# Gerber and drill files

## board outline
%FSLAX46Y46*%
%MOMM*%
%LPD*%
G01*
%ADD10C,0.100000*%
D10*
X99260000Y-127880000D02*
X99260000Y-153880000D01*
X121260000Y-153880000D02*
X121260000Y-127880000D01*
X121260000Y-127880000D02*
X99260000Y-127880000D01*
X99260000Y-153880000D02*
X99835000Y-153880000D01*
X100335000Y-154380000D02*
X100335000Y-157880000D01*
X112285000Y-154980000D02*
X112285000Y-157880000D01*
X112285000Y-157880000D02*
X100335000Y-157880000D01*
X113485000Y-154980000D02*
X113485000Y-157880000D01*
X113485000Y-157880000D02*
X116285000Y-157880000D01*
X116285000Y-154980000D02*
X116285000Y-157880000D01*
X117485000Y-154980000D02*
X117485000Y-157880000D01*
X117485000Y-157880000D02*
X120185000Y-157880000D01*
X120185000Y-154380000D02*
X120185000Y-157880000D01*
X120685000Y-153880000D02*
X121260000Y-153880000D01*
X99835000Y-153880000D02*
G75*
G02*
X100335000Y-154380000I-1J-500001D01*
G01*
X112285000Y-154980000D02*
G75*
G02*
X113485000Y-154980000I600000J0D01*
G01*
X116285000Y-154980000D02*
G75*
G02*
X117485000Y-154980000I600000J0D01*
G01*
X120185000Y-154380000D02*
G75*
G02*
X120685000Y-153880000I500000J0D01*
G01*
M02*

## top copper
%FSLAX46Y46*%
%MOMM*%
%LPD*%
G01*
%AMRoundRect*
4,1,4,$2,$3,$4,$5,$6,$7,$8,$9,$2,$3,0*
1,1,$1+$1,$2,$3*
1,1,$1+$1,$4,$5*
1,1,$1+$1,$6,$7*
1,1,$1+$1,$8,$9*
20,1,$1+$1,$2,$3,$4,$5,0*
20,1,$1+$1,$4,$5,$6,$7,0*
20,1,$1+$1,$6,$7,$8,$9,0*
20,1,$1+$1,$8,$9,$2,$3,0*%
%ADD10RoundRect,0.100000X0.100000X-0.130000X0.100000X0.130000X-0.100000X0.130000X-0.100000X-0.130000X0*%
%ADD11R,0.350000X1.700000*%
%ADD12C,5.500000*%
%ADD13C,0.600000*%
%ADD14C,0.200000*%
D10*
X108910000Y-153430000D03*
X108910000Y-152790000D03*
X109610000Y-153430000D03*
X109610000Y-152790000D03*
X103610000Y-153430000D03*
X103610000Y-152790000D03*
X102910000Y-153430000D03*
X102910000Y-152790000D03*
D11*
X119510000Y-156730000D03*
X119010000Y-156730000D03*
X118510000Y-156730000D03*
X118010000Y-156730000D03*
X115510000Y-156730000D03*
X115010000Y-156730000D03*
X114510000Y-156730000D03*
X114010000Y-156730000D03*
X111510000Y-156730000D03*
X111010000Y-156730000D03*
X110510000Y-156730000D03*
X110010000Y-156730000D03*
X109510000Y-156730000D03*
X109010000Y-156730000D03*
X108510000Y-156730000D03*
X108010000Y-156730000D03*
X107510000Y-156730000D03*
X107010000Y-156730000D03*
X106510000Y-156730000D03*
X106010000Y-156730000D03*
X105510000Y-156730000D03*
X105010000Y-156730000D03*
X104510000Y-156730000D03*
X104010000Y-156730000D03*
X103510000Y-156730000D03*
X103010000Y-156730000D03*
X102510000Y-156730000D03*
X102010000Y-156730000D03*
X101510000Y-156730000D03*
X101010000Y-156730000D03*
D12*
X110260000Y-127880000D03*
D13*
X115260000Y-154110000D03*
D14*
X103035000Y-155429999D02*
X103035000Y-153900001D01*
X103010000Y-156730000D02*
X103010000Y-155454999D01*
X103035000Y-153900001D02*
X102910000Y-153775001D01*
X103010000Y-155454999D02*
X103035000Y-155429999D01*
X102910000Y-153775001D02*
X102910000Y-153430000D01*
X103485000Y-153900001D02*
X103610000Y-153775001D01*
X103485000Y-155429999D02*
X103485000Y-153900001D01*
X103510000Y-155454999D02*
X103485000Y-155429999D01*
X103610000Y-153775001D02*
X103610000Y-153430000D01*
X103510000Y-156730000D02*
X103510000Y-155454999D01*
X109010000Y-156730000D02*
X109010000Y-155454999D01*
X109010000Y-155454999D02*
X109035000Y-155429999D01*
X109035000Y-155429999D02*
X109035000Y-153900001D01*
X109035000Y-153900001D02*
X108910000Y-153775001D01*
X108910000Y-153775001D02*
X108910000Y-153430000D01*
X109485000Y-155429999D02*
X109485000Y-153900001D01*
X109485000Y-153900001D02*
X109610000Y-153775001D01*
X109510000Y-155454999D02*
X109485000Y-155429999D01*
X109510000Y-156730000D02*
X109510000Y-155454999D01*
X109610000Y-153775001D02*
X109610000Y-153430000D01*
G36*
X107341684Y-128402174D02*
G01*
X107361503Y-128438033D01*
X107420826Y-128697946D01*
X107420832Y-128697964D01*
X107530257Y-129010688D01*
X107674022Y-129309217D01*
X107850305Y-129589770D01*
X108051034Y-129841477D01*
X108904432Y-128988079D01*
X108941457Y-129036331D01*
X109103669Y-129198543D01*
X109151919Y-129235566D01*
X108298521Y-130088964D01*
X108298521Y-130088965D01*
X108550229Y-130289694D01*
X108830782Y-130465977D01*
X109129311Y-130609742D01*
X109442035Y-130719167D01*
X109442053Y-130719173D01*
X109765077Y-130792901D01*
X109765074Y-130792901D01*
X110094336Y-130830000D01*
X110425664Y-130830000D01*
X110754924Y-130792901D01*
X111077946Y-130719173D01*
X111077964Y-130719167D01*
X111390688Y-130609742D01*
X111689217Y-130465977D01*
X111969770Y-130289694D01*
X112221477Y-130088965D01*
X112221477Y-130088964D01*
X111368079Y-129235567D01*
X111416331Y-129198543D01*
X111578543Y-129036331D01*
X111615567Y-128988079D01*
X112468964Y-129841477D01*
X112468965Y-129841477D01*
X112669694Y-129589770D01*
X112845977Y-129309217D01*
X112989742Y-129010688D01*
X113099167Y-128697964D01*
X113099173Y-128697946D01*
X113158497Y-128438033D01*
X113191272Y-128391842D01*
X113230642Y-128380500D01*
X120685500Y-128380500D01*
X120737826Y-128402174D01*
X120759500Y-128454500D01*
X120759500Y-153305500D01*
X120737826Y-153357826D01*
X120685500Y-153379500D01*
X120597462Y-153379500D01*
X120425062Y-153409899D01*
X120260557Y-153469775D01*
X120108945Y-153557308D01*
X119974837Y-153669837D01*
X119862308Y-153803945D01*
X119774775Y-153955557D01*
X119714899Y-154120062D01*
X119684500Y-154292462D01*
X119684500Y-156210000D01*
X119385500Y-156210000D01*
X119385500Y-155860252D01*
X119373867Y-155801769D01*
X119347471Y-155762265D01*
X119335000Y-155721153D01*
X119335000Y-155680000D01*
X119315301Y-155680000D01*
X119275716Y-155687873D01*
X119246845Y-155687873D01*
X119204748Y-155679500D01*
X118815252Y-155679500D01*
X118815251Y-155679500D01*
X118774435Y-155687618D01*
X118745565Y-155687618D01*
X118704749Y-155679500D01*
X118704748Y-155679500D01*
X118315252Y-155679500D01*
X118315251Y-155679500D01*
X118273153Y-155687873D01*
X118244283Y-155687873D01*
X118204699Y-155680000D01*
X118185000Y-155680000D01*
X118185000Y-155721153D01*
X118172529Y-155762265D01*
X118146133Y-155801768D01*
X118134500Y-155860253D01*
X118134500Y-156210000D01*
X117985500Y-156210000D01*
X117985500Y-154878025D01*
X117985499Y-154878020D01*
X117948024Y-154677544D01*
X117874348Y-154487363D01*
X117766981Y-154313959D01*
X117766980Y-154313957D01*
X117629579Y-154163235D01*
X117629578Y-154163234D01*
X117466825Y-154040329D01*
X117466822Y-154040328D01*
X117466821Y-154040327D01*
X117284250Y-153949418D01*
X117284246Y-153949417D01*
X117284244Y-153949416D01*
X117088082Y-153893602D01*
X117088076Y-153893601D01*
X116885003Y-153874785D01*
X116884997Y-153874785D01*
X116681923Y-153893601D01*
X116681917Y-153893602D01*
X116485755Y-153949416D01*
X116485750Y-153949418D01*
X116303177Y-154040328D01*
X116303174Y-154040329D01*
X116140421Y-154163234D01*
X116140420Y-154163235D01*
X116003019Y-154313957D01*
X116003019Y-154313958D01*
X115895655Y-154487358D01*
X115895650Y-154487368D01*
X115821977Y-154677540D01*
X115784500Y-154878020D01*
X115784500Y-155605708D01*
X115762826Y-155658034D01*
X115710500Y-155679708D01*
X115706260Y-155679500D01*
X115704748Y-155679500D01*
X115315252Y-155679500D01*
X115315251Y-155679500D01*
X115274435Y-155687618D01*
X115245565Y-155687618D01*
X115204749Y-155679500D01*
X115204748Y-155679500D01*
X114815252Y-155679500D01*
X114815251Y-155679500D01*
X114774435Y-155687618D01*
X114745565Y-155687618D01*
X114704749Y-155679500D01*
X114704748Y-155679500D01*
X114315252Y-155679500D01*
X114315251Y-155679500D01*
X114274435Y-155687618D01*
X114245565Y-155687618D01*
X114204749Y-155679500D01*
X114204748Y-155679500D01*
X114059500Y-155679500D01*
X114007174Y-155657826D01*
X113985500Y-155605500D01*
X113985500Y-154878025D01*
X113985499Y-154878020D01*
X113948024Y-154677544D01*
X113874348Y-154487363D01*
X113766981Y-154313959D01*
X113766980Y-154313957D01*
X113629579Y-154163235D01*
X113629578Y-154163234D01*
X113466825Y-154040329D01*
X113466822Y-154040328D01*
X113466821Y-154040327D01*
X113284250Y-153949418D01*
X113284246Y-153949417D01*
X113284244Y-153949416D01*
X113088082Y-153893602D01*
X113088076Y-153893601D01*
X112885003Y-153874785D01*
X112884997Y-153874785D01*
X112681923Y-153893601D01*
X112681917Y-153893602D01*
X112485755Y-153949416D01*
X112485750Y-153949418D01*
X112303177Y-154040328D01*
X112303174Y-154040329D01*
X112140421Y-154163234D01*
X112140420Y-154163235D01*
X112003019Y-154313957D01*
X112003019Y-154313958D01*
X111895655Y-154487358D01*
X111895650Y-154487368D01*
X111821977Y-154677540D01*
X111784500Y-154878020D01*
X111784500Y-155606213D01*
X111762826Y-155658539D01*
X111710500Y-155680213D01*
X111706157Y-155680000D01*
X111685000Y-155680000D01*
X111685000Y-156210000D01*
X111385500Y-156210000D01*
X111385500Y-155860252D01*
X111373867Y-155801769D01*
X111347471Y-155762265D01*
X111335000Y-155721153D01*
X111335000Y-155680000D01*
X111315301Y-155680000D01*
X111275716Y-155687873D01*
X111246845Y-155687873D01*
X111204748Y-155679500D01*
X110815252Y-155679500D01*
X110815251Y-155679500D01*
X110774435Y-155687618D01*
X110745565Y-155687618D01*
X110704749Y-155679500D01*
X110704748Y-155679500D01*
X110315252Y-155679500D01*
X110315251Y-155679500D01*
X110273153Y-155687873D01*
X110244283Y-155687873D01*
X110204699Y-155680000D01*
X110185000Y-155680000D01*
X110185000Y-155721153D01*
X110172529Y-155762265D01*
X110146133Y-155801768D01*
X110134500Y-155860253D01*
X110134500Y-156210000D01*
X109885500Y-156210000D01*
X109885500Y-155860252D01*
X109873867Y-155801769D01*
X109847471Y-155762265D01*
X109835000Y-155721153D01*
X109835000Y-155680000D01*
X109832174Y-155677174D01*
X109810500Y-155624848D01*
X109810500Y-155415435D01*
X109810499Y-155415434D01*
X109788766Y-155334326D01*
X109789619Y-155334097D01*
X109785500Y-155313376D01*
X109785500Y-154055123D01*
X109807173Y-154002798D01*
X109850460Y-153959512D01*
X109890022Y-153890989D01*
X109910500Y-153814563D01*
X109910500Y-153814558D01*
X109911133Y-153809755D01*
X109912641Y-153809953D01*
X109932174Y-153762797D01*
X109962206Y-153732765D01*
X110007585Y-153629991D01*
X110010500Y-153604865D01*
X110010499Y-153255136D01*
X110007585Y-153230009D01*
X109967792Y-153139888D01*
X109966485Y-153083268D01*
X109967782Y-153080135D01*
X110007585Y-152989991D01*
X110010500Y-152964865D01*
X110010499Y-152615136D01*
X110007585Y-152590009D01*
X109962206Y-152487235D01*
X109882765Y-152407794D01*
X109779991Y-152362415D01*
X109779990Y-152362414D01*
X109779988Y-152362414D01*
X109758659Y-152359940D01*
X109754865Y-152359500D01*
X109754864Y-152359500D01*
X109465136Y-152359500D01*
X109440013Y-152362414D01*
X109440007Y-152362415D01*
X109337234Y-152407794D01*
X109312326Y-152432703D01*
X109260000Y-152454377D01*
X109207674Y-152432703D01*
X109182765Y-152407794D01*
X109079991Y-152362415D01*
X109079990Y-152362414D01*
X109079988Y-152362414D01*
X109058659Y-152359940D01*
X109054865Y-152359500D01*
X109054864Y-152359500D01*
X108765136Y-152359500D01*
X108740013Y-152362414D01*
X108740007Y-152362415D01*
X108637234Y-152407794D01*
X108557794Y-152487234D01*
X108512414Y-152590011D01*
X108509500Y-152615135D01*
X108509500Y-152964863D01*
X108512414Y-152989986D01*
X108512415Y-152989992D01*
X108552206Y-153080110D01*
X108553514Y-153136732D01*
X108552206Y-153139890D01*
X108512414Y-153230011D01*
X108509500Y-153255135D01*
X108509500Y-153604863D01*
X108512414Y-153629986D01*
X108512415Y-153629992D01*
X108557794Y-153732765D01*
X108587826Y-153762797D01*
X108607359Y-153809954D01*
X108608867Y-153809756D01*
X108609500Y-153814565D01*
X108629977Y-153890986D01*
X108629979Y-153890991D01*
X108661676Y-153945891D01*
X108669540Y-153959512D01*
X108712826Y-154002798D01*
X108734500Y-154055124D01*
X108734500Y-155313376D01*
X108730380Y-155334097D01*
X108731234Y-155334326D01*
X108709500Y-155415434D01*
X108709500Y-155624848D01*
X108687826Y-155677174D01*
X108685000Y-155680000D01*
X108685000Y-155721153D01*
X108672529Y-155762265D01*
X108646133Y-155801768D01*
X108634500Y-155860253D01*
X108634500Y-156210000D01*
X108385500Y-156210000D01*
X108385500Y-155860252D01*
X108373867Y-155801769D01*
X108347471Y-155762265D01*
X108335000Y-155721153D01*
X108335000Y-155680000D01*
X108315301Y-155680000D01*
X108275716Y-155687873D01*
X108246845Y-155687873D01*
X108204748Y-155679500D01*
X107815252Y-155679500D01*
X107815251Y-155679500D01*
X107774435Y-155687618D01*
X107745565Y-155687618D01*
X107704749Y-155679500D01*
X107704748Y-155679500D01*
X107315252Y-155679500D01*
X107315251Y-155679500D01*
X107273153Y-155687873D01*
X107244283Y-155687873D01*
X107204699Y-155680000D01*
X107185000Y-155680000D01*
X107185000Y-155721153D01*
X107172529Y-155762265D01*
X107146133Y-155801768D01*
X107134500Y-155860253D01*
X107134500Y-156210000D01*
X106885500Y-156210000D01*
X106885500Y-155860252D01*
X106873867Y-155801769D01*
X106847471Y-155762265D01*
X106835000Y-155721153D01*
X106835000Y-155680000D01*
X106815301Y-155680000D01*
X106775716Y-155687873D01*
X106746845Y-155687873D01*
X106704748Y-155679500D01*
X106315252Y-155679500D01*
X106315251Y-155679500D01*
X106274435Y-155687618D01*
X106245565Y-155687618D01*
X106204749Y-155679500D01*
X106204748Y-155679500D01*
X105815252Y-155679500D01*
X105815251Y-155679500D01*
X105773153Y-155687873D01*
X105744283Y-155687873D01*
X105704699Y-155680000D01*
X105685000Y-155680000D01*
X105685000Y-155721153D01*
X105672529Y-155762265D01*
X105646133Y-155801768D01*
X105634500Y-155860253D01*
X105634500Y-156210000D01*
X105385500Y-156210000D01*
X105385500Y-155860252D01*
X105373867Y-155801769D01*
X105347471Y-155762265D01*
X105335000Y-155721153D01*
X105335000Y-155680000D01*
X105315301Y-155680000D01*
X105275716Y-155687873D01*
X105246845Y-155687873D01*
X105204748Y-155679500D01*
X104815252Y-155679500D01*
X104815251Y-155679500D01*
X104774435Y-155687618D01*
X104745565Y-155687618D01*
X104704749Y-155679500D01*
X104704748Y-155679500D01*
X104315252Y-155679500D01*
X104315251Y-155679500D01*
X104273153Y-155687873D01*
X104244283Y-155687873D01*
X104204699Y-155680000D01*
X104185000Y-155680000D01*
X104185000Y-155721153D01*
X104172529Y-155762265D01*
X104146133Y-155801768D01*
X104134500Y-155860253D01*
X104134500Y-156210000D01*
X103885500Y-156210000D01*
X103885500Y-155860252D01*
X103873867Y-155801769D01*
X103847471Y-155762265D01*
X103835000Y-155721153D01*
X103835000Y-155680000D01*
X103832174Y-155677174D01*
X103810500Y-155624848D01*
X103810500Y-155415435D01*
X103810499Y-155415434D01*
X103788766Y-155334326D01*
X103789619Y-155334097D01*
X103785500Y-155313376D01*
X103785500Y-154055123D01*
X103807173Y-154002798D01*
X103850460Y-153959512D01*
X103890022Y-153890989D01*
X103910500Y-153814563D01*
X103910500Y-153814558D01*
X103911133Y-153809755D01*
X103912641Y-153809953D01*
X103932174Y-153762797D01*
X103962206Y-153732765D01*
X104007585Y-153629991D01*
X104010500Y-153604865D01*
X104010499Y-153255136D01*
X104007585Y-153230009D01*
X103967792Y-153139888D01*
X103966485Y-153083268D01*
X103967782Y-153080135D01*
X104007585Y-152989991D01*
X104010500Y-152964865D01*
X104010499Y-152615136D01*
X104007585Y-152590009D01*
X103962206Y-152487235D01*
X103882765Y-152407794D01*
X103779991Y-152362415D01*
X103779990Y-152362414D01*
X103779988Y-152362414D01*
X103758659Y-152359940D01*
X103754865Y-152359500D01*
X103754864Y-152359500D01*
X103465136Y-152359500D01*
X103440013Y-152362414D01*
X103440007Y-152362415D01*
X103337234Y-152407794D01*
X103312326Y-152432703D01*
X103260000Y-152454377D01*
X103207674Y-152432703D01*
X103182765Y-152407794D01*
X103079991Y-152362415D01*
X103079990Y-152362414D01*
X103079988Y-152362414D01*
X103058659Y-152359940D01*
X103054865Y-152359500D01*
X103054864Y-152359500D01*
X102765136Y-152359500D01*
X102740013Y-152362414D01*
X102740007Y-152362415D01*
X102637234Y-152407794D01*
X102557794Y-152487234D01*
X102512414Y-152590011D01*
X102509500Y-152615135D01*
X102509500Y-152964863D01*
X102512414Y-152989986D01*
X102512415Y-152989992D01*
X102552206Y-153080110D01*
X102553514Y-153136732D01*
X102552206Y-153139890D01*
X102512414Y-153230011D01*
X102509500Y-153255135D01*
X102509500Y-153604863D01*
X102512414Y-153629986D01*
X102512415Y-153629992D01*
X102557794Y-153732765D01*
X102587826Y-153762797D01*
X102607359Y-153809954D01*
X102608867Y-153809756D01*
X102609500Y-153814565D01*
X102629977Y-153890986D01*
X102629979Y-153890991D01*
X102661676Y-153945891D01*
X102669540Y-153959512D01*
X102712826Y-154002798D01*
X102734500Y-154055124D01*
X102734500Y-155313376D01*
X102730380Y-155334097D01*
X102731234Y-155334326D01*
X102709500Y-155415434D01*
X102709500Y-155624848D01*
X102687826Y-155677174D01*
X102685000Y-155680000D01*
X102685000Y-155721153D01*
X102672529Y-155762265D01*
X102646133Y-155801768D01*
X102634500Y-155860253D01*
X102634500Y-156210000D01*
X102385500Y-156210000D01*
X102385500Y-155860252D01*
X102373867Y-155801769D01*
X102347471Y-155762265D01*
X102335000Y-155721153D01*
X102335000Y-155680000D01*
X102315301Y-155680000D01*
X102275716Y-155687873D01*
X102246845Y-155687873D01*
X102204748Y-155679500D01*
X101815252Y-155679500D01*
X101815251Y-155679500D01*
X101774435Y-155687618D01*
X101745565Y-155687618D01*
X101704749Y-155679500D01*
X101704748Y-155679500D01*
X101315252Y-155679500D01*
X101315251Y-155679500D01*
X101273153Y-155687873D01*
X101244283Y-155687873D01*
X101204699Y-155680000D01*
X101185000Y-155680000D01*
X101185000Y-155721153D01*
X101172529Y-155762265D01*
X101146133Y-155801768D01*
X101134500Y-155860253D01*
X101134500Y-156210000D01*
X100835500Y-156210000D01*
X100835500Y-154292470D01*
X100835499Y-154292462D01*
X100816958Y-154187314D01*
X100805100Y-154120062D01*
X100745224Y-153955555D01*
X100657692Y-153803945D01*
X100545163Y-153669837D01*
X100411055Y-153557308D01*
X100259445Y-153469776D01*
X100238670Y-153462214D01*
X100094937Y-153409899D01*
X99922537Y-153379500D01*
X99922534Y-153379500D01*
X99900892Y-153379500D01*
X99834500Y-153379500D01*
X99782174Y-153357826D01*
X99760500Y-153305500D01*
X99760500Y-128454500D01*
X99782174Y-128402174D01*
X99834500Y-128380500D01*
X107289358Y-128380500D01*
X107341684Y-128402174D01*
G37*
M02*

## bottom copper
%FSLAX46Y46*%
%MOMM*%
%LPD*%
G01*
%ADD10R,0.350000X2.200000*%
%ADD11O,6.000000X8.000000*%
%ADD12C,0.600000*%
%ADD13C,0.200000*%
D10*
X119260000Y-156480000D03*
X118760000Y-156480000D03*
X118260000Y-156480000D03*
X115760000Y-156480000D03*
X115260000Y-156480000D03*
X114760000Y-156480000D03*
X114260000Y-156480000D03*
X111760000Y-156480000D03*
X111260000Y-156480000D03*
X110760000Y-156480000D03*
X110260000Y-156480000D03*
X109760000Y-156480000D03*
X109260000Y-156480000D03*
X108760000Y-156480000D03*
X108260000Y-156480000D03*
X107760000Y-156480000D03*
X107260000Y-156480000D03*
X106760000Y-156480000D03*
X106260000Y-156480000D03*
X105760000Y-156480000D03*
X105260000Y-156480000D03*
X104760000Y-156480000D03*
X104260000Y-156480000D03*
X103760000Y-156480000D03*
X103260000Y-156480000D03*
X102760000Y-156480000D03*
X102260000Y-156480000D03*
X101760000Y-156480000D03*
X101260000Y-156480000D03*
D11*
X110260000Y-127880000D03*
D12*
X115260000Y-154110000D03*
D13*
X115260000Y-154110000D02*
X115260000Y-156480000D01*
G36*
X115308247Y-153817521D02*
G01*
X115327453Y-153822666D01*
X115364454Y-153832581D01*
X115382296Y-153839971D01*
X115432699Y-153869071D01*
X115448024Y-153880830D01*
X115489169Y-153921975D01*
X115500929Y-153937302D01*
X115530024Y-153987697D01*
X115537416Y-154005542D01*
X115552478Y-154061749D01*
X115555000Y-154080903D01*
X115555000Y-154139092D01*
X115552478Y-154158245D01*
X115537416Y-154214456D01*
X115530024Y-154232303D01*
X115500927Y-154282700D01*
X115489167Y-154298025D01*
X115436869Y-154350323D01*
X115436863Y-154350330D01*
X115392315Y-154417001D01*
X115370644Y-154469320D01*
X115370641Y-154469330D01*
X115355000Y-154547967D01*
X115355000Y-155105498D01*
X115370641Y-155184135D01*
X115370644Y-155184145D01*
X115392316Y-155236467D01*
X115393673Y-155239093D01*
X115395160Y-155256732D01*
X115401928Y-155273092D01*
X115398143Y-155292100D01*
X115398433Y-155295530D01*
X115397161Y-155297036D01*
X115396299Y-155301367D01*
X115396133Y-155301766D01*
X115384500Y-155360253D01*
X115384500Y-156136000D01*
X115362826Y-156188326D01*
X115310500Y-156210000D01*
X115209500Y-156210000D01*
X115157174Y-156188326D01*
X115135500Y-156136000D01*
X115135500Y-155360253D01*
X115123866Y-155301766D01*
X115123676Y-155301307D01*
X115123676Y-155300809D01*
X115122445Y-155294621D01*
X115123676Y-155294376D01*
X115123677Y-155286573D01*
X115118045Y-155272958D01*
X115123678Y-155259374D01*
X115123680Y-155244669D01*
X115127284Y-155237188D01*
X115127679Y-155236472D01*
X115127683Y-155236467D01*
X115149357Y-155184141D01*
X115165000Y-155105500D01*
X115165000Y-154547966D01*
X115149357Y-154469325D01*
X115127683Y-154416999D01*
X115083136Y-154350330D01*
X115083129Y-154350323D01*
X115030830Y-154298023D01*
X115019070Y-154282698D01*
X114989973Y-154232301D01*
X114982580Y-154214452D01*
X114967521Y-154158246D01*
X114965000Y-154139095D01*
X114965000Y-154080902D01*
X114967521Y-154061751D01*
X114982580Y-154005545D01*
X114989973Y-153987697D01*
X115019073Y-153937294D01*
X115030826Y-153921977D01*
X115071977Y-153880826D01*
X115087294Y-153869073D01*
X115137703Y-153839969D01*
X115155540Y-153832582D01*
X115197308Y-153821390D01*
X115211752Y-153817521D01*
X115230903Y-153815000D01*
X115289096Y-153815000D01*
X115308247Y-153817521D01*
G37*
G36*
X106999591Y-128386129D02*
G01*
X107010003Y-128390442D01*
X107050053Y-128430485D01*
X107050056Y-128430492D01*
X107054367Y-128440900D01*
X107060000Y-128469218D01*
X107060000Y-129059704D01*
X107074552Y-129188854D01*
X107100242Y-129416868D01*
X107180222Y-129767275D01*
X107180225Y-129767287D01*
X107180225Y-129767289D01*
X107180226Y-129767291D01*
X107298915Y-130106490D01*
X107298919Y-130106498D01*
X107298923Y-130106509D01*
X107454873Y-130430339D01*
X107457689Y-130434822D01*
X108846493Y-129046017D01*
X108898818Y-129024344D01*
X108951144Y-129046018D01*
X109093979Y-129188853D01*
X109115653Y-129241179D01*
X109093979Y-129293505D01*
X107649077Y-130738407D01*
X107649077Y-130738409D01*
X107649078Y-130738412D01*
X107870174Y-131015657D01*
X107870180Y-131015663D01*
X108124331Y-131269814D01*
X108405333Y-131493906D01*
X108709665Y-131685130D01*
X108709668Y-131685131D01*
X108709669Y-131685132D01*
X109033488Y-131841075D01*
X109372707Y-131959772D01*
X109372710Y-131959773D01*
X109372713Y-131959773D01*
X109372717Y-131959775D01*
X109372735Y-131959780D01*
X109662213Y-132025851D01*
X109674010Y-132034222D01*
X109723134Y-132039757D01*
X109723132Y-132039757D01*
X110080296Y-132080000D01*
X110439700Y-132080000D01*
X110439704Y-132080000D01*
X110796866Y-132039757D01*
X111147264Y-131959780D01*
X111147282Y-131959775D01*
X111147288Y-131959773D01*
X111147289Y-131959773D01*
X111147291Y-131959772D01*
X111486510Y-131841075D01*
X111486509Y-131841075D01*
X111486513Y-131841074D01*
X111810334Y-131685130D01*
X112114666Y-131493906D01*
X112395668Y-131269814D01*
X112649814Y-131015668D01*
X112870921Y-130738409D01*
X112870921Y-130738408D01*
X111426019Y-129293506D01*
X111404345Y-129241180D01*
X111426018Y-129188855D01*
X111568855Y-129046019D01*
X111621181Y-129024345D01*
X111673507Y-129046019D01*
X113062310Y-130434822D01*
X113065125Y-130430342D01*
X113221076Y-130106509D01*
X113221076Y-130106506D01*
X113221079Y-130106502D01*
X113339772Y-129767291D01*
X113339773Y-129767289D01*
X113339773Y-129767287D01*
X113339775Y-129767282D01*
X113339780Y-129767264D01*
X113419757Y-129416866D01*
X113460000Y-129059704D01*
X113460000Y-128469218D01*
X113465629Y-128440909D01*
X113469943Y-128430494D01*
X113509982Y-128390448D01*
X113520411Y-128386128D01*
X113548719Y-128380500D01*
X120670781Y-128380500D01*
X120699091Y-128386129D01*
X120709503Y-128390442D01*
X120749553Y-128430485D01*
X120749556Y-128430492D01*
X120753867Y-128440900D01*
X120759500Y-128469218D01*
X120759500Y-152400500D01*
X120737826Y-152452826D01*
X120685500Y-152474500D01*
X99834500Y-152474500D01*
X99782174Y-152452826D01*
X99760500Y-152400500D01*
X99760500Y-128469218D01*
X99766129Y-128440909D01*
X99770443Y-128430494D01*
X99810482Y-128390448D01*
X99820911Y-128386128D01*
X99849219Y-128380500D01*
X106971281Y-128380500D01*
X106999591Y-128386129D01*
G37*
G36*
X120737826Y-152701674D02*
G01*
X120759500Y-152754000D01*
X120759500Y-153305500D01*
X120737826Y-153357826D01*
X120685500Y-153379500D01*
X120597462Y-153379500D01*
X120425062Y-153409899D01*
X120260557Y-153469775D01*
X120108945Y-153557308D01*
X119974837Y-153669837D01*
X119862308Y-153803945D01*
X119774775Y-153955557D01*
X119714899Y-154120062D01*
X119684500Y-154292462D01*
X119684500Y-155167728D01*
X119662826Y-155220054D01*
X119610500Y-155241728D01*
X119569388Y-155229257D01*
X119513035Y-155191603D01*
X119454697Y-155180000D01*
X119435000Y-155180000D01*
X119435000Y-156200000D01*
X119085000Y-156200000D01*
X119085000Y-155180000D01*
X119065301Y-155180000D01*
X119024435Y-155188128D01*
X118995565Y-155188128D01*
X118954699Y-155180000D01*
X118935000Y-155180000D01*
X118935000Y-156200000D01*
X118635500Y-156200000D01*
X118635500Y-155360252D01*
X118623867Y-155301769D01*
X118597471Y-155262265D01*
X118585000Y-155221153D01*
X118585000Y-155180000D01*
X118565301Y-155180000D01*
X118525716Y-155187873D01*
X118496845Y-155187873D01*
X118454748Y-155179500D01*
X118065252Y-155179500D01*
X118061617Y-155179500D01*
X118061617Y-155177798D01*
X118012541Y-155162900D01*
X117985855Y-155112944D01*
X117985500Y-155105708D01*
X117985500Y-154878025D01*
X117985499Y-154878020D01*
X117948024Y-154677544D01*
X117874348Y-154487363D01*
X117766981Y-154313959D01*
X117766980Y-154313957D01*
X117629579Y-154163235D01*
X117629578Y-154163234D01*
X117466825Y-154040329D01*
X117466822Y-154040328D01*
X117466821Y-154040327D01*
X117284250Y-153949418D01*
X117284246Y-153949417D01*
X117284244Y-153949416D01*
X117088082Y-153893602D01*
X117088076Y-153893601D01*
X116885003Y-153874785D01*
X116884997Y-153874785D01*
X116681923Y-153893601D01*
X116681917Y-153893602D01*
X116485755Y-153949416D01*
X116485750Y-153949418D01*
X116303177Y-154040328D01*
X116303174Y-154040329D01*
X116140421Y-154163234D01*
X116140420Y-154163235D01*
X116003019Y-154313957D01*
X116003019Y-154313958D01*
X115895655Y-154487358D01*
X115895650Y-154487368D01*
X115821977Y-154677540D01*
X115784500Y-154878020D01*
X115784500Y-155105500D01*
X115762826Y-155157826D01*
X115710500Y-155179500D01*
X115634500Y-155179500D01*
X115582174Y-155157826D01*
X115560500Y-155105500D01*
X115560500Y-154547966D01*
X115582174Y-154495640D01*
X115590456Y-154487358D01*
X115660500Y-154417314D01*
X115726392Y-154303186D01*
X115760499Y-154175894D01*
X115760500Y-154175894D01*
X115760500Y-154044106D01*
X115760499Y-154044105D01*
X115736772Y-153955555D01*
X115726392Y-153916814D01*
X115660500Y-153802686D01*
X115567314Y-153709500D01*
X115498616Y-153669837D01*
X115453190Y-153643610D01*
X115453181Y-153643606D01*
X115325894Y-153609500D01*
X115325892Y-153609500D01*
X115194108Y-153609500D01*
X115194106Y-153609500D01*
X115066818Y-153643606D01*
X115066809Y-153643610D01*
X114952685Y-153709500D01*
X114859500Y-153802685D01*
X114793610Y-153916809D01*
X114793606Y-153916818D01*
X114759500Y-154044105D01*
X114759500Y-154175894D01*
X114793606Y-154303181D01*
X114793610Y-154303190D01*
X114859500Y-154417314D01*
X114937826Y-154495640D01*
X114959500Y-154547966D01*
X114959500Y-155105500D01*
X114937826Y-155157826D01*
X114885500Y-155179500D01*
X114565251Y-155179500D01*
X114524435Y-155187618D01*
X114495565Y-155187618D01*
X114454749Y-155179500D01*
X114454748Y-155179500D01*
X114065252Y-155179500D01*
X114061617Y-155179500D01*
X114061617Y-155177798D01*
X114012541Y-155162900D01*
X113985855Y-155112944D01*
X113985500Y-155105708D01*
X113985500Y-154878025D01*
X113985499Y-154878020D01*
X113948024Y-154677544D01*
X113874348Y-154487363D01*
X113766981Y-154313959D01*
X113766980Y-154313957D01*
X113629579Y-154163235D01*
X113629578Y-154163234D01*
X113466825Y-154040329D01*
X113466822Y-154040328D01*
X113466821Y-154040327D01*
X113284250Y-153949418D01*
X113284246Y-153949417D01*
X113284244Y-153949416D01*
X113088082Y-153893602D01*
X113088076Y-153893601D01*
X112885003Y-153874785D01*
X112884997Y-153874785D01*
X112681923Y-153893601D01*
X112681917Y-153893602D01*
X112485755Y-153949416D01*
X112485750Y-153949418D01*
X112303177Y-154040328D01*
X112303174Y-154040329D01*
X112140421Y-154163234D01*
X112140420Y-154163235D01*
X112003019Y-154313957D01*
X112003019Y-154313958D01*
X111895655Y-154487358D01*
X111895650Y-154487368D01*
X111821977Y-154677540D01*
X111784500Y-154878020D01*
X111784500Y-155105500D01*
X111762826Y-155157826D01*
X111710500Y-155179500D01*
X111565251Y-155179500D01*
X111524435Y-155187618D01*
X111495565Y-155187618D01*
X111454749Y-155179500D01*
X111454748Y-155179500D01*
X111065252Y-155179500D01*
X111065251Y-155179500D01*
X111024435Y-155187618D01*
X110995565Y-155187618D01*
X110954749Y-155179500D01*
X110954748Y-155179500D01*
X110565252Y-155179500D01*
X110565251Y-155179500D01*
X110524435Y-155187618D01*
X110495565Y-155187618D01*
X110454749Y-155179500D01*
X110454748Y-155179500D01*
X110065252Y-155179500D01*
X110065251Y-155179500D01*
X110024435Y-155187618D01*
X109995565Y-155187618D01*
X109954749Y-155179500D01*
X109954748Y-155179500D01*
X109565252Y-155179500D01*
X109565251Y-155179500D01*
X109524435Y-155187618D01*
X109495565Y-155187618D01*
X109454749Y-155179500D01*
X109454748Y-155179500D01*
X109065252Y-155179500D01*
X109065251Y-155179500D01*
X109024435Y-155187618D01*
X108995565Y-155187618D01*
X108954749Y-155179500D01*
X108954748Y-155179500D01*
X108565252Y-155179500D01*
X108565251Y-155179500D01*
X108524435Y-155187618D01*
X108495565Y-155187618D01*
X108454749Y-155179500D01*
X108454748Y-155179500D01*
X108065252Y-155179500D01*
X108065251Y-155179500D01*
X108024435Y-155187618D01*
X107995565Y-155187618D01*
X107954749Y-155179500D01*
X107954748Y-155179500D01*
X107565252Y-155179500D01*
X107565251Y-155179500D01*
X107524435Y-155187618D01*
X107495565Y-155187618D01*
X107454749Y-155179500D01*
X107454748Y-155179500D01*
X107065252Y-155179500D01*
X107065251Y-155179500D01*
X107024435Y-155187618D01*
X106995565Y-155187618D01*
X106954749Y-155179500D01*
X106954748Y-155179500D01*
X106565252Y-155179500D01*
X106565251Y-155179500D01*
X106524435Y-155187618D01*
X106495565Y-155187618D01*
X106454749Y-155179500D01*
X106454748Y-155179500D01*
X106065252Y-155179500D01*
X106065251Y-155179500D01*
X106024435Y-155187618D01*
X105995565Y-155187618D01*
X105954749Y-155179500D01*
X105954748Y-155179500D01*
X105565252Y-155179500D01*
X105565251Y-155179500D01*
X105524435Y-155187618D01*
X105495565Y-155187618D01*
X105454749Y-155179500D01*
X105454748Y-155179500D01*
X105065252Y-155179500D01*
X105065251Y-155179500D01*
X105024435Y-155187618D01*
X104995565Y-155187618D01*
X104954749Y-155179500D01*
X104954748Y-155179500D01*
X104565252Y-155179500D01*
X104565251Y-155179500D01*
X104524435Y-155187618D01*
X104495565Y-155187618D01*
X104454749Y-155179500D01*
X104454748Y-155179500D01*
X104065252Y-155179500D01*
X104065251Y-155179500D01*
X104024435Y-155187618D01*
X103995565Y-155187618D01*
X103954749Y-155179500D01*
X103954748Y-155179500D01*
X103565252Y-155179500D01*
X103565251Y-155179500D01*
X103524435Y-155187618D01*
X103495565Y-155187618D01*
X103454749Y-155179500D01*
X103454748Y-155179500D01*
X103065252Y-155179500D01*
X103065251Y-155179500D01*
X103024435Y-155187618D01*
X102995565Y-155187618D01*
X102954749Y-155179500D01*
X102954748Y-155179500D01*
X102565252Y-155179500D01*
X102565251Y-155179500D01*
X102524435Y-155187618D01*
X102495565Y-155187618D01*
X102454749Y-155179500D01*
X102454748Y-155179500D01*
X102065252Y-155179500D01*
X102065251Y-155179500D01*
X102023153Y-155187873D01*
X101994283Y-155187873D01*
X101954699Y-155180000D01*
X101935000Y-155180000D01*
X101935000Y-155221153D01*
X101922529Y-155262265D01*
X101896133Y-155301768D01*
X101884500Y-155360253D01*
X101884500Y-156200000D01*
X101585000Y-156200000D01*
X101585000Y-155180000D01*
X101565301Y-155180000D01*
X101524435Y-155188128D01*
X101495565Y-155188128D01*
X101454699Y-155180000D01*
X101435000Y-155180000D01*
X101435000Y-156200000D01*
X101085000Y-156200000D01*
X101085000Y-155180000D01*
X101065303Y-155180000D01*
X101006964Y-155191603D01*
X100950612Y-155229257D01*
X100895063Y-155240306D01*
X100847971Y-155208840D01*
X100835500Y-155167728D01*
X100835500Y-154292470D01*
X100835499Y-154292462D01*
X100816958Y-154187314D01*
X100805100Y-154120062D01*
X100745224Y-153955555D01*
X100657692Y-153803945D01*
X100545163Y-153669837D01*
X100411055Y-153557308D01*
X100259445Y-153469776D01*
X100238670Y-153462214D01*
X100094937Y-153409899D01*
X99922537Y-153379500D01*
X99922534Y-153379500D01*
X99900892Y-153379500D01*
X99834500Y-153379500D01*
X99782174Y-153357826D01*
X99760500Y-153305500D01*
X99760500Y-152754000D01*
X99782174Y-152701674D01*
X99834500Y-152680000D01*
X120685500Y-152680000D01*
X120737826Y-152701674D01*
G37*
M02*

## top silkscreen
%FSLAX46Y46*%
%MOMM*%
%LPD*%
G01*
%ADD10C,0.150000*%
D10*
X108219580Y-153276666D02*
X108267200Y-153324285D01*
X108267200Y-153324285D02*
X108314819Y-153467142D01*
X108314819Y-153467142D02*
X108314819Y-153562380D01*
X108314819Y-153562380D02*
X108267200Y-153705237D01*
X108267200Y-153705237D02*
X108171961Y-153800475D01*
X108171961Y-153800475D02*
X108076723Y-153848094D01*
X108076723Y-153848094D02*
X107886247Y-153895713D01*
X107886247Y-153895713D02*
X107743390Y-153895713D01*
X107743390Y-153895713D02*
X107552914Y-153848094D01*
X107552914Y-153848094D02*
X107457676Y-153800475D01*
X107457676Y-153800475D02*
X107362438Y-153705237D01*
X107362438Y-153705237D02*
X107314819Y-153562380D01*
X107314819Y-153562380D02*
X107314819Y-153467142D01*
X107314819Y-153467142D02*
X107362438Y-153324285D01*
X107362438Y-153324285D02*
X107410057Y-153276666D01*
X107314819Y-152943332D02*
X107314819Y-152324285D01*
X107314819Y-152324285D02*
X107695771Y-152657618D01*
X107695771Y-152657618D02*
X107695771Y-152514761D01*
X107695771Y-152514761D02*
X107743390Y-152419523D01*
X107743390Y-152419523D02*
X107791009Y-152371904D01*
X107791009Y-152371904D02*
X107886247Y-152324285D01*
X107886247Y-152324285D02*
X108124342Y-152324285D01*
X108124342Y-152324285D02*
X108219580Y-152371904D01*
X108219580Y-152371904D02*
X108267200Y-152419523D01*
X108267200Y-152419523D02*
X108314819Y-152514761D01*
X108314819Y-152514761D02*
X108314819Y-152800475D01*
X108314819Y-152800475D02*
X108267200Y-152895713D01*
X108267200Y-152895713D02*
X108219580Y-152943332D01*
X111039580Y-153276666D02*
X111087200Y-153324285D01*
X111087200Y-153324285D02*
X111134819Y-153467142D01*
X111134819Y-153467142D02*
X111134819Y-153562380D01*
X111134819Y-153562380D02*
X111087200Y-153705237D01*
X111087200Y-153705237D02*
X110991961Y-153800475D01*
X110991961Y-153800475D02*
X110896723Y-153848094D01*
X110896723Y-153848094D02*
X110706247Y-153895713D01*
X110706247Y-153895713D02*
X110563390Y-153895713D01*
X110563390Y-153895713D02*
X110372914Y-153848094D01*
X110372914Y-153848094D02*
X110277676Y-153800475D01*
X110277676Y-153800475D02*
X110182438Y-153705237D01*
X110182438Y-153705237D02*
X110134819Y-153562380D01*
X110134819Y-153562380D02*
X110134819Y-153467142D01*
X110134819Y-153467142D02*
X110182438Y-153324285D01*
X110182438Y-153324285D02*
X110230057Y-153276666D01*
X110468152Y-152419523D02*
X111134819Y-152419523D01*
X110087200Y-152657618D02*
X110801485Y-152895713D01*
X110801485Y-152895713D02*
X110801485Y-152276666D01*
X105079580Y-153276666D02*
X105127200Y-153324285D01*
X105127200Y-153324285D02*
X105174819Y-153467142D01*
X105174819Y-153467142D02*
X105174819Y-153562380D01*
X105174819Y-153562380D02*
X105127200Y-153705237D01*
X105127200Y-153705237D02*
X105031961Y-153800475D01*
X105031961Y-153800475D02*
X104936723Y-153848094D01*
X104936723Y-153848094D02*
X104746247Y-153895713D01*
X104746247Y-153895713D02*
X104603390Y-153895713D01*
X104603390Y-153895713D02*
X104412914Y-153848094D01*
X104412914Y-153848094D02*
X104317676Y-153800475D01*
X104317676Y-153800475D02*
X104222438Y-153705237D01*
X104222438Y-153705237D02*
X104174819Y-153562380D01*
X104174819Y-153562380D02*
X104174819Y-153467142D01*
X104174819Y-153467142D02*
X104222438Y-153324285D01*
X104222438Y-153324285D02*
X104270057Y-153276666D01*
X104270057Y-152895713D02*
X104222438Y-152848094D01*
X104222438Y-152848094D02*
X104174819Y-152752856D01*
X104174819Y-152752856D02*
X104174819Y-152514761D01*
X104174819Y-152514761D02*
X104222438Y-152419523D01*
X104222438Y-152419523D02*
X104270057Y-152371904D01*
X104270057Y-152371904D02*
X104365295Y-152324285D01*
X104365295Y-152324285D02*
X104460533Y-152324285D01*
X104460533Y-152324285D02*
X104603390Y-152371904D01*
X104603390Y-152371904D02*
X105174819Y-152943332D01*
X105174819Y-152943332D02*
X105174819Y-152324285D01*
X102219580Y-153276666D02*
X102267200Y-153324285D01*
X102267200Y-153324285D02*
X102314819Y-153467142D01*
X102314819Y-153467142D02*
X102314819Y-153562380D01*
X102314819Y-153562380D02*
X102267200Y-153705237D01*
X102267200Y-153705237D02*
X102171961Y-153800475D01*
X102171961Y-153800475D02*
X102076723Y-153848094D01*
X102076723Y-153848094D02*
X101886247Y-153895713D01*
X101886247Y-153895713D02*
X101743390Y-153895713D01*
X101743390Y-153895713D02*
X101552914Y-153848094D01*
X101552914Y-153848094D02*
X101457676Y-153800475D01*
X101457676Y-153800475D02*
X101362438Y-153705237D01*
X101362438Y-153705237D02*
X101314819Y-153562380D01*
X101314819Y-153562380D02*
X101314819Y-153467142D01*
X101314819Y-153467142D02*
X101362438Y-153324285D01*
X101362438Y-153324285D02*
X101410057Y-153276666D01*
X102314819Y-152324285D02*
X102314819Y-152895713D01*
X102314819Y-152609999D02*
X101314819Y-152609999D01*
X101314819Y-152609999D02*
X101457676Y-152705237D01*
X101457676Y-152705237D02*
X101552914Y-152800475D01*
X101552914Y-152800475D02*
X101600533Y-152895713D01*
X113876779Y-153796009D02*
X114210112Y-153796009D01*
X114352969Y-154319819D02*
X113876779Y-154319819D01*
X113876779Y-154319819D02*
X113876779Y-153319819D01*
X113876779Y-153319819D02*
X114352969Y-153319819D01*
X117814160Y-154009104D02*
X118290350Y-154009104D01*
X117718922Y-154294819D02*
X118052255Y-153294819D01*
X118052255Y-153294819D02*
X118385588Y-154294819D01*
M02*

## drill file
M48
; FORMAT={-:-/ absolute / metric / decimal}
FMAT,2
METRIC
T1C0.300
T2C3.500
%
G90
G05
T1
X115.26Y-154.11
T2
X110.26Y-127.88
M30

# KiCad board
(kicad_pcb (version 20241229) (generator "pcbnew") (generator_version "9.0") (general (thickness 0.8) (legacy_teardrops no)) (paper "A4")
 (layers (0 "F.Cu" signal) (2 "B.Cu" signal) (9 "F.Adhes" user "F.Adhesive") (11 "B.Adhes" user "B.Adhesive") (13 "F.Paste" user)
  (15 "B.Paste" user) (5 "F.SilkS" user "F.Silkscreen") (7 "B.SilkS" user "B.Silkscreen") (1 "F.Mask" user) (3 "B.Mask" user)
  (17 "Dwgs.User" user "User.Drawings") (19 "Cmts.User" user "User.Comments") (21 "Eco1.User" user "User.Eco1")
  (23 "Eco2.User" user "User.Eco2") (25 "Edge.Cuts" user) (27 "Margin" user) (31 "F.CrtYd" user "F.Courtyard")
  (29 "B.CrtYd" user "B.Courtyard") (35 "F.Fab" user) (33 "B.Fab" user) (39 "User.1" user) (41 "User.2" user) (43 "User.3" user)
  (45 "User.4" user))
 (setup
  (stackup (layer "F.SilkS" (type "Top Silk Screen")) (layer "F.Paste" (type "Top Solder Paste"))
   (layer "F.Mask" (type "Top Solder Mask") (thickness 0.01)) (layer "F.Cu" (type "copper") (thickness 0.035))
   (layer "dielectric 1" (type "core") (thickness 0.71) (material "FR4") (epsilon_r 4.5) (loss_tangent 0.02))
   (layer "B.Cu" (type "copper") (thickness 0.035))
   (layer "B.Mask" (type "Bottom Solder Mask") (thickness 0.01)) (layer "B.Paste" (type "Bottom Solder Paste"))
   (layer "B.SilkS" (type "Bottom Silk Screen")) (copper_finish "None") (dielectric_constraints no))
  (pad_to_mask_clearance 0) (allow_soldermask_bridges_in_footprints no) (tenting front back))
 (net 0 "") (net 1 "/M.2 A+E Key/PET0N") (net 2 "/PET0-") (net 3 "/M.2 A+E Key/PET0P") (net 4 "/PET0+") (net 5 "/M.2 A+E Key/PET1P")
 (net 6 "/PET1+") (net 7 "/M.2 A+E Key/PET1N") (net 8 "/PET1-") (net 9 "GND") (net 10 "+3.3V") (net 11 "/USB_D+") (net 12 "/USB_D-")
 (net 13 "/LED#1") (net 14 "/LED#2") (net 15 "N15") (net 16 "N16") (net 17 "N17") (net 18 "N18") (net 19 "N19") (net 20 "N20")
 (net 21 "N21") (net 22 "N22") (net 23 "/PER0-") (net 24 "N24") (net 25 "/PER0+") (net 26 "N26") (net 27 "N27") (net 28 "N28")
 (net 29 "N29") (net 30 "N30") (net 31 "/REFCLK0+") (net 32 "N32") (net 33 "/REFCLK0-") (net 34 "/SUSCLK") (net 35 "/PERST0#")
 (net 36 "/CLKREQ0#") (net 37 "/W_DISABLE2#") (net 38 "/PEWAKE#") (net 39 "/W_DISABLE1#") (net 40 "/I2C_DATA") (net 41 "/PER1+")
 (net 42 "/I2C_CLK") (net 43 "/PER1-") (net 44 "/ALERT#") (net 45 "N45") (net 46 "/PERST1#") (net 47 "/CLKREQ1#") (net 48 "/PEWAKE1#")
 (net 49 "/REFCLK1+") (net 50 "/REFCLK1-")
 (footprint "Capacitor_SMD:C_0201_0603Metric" (layer "F.Cu") (at 108.91 153.11 90)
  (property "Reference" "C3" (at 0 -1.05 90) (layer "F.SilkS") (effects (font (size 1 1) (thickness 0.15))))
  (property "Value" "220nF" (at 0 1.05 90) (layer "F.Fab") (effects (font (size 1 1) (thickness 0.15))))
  (pad "" smd roundrect (at -0.345 0 90) (size 0.318 0.36) (layers "F.Paste") (roundrect_rratio 0.25))
  (pad "" smd roundrect (at 0.345 0 90) (size 0.318 0.36) (layers "F.Paste") (roundrect_rratio 0.25))
  (pad "1" smd roundrect (at -0.32 0 90) (size 0.46 0.4) (layers "F.Cu" "F.Mask") (roundrect_rratio 0.25) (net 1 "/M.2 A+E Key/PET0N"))
  (pad "2" smd roundrect (at 0.32 0 90) (size 0.46 0.4) (layers "F.Cu" "F.Mask") (roundrect_rratio 0.25) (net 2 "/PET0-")))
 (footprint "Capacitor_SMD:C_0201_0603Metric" (layer "F.Cu") (at 109.61 153.11 90)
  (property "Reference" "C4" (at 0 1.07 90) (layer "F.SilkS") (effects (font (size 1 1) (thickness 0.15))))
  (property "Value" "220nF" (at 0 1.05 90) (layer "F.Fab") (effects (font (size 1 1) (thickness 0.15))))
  (pad "" smd roundrect (at -0.345 0 90) (size 0.318 0.36) (layers "F.Paste") (roundrect_rratio 0.25))
  (pad "" smd roundrect (at 0.345 0 90) (size 0.318 0.36) (layers "F.Paste") (roundrect_rratio 0.25))
  (pad "1" smd roundrect (at -0.32 0 90) (size 0.46 0.4) (layers "F.Cu" "F.Mask") (roundrect_rratio 0.25) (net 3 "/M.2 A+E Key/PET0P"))
  (pad "2" smd roundrect (at 0.32 0 90) (size 0.46 0.4) (layers "F.Cu" "F.Mask") (roundrect_rratio 0.25) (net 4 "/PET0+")))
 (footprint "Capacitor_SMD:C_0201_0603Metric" (layer "F.Cu") (at 103.61 153.11 90)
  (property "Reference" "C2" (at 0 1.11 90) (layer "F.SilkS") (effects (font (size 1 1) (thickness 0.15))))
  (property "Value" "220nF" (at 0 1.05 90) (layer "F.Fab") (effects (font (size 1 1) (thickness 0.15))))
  (pad "" smd roundrect (at -0.345 0 90) (size 0.318 0.36) (layers "F.Paste") (roundrect_rratio 0.25))
  (pad "" smd roundrect (at 0.345 0 90) (size 0.318 0.36) (layers "F.Paste") (roundrect_rratio 0.25))
  (pad "1" smd roundrect (at -0.32 0 90) (size 0.46 0.4) (layers "F.Cu" "F.Mask") (roundrect_rratio 0.25) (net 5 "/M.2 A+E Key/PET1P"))
  (pad "2" smd roundrect (at 0.32 0 90) (size 0.46 0.4) (layers "F.Cu" "F.Mask") (roundrect_rratio 0.25) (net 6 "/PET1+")))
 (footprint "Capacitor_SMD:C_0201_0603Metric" (layer "F.Cu") (at 102.91 153.11 90)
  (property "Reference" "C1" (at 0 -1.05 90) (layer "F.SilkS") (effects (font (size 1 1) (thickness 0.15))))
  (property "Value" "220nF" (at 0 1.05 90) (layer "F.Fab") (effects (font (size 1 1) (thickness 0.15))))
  (pad "" smd roundrect (at -0.345 0 90) (size 0.318 0.36) (layers "F.Paste") (roundrect_rratio 0.25))
  (pad "" smd roundrect (at 0.345 0 90) (size 0.318 0.36) (layers "F.Paste") (roundrect_rratio 0.25))
  (pad "1" smd roundrect (at -0.32 0 90) (size 0.46 0.4) (layers "F.Cu" "F.Mask") (roundrect_rratio 0.25) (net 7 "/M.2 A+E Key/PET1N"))
  (pad "2" smd roundrect (at 0.32 0 90) (size 0.46 0.4) (layers "F.Cu" "F.Mask") (roundrect_rratio 0.25) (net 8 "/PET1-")))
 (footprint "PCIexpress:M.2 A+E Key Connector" (layer "F.Cu") (at 110.26 156.77)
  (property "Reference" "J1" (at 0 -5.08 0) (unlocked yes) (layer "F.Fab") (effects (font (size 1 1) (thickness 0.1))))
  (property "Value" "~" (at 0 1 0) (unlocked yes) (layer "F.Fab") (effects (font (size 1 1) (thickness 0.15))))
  (fp_line (start -11 -2.89) (end -10.425 -2.89) (stroke (width 0.1) (type default)) (layer "Edge.Cuts"))
  (fp_line (start -9.925 -2.39) (end -9.925 1.11) (stroke (width 0.1) (type default)) (layer "Edge.Cuts"))
  (fp_line (start 2.025 -1.79) (end 2.025 1.11) (stroke (width 0.1) (type default)) (layer "Edge.Cuts"))
  (fp_line (start 2.025 1.11) (end -9.925 1.11) (stroke (width 0.1) (type default)) (layer "Edge.Cuts"))
  (fp_line (start 3.225 -1.79) (end 3.225 1.11) (stroke (width 0.1) (type default)) (layer "Edge.Cuts"))
  (fp_line (start 3.225 1.11) (end 6.025 1.11) (stroke (width 0.1) (type default)) (layer "Edge.Cuts"))
  (fp_line (start 6.025 -1.79) (end 6.025 1.11) (stroke (width 0.1) (type default)) (layer "Edge.Cuts"))
  (fp_line (start 7.225 -1.79) (end 7.225 1.11) (stroke (width 0.1) (type default)) (layer "Edge.Cuts"))
  (fp_line (start 7.225 1.11) (end 9.925 1.11) (stroke (width 0.1) (type default)) (layer "Edge.Cuts"))
  (fp_line (start 9.925 -2.39) (end 9.925 1.11) (stroke (width 0.1) (type default)) (layer "Edge.Cuts"))
  (fp_line (start 10.425 -2.89) (end 11 -2.89) (stroke (width 0.1) (type default)) (layer "Edge.Cuts"))
  (fp_arc (start -10.425 -2.89) (mid -10.071447 -2.743553) (end -9.925 -2.39) (stroke (width 0.1) (type default)) (layer "Edge.Cuts"))
  (fp_arc (start 2.025 -1.79) (mid 2.625 -2.39) (end 3.225 -1.79) (stroke (width 0.1) (type default)) (layer "Edge.Cuts"))
  (fp_arc (start 6.025 -1.79) (mid 6.625 -2.39) (end 7.225 -1.79) (stroke (width 0.1) (type default)) (layer "Edge.Cuts"))
  (fp_arc (start 9.925 -2.39) (mid 10.071447 -2.743553) (end 10.425 -2.89) (stroke (width 0.1) (type default)) (layer "Edge.Cuts"))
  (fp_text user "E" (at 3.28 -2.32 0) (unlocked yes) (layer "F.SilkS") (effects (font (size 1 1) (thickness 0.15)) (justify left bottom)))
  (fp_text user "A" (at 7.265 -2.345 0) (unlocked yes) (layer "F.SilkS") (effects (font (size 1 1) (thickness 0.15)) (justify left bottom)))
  (pad "1" smd rect (at 9.25 -0.04 180) (size 0.35 1.7) (layers "F.Cu") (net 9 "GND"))
  (pad "2" smd rect (at 9 -0.29 180) (size 0.35 2.2) (layers "B.Cu") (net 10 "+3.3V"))
  (pad "3" smd rect (at 8.75 -0.04 180) (size 0.35 1.7) (layers "F.Cu") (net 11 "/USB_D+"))
  (pad "4" smd rect (at 8.5 -0.29 180) (size 0.35 2.2) (layers "B.Cu") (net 10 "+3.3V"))
  (pad "5" smd rect (at 8.25 -0.04 180) (size 0.35 1.7) (layers "F.Cu") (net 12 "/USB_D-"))
  (pad "6" smd rect (at 8 -0.29 180) (size 0.35 2.2) (layers "B.Cu") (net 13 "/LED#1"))
  (pad "7" smd rect (at 7.75 -0.04 180) (size 0.35 1.7) (layers "F.Cu") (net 9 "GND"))
  (pad "16" smd rect (at 5.5 -0.29 180) (size 0.35 2.2) (layers "B.Cu") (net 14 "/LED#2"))
  (pad "17" smd rect (at 5.25 -0.04 180) (size 0.35 1.7) (layers "F.Cu") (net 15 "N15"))
  (pad "18" smd rect (at 5 -0.29 180) (size 0.35 2.2) (layers "B.Cu") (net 9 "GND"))
  (pad "19" smd rect (at 4.75 -0.04 180) (size 0.35 1.7) (layers "F.Cu") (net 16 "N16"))
  (pad "20" smd rect (at 4.5 -0.29 180) (size 0.35 2.2) (layers "B.Cu") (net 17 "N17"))
  (pad "21" smd rect (at 4.25 -0.04 180) (size 0.35 1.7) (layers "F.Cu") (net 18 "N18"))
  (pad "22" smd rect (at 4 -0.29 180) (size 0.35 2.2) (layers "B.Cu") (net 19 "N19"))
  (pad "23" smd rect (at 3.75 -0.04 180) (size 0.35 1.7) (layers "F.Cu") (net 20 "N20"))
  (pad "32" smd rect (at 1.5 -0.29 180) (size 0.35 2.2) (layers "B.Cu") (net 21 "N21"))
  (pad "33" smd rect (at 1.25 -0.04 180) (size 0.35 1.7) (layers "F.Cu") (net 9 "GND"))
  (pad "34" smd rect (at 1 -0.29 180) (size 0.35 2.2) (layers "B.Cu") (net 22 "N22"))
  (pad "35" smd rect (at 0.75 -0.04 180) (size 0.35 1.7) (layers "F.Cu") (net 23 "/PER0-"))
  (pad "36" smd rect (at 0.5 -0.29 180) (size 0.35 2.2) (layers "B.Cu") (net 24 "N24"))
  (pad "37" smd rect (at 0.25 -0.04 180) (size 0.35 1.7) (layers "F.Cu") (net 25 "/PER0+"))
  (pad "38" smd rect (at 0 -0.29 180) (size 0.35 2.2) (layers "B.Cu") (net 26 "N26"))
  (pad "39" smd rect (at -0.25 -0.04 180) (size 0.35 1.7) (layers "F.Cu") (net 9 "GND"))
  (pad "40" smd rect (at -0.5 -0.29 180) (size 0.35 2.2) (layers "B.Cu") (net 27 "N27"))
  (pad "41" smd rect (at -0.75 -0.04 180) (size 0.35 1.7) (layers "F.Cu") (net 3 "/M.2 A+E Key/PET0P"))
  (pad "42" smd rect (at -1 -0.29 180) (size 0.35 2.2) (layers "B.Cu") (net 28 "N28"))
  (pad "43" smd rect (at -1.25 -0.04 180) (size 0.35 1.7) (layers "F.Cu") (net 1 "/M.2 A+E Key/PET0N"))
  (pad "44" smd rect (at -1.5 -0.29 180) (size 0.35 2.2) (layers "B.Cu") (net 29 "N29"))
  (pad "45" smd rect (at -1.75 -0.04 180) (size 0.35 1.7) (layers "F.Cu") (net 9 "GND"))
  (pad "46" smd rect (at -2 -0.29 180) (size 0.35 2.2) (layers "B.Cu") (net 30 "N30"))
  (pad "47" smd rect (at -2.25 -0.04 180) (size 0.35 1.7) (layers "F.Cu") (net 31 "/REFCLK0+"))
  (pad "48" smd rect (at -2.5 -0.29 180) (size 0.35 2.2) (layers "B.Cu") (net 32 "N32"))
  (pad "49" smd rect (at -2.75 -0.04 180) (size 0.35 1.7) (layers "F.Cu") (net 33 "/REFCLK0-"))
  (pad "50" smd rect (at -3 -0.29 180) (size 0.35 2.2) (layers "B.Cu") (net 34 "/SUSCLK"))
  (pad "51" smd rect (at -3.25 -0.04 180) (size 0.35 1.7) (layers "F.Cu") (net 9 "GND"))
  (pad "52" smd rect (at -3.5 -0.29 180) (size 0.35 2.2) (layers "B.Cu") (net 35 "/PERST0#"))
  (pad "53" smd rect (at -3.75 -0.04 180) (size 0.35 1.7) (layers "F.Cu") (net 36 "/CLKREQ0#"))
  (pad "54" smd rect (at -4 -0.29 180) (size 0.35 2.2) (layers "B.Cu") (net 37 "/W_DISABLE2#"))
  (pad "55" smd rect (at -4.25 -0.04 180) (size 0.35 1.7) (layers "F.Cu") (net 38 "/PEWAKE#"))
  (pad "56" smd rect (at -4.5 -0.29 180) (size 0.35 2.2) (layers "B.Cu") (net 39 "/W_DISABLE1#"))
  (pad "57" smd rect (at -4.75 -0.04 180) (size 0.35 1.7) (layers "F.Cu") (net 9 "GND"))
  (pad "58" smd rect (at -5 -0.29 180) (size 0.35 2.2) (layers "B.Cu") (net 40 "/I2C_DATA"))
  (pad "59" smd rect (at -5.25 -0.04 180) (size 0.35 1.7) (layers "F.Cu") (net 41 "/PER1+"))
  (pad "60" smd rect (at -5.5 -0.29 180) (size 0.35 2.2) (layers "B.Cu") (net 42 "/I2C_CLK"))
  (pad "61" smd rect (at -5.75 -0.04 180) (size 0.35 1.7) (layers "F.Cu") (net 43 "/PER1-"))
  (pad "62" smd rect (at -6 -0.29 180) (size 0.35 2.2) (layers "B.Cu") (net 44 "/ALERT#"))
  (pad "63" smd rect (at -6.25 -0.04 180) (size 0.35 1.7) (layers "F.Cu") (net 9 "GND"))
  (pad "64" smd rect (at -6.5 -0.29 180) (size 0.35 2.2) (layers "B.Cu") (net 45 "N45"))
  (pad "65" smd rect (at -6.75 -0.04 180) (size 0.35 1.7) (layers "F.Cu") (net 5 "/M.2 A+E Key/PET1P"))
  (pad "66" smd rect (at -7 -0.29 180) (size 0.35 2.2) (layers "B.Cu") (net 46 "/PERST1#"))
  (pad "67" smd rect (at -7.25 -0.04 180) (size 0.35 1.7) (layers "F.Cu") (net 7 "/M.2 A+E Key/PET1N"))
  (pad "68" smd rect (at -7.5 -0.29 180) (size 0.35 2.2) (layers "B.Cu") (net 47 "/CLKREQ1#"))
  (pad "69" smd rect (at -7.75 -0.04 180) (size 0.35 1.7) (layers "F.Cu") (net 9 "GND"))
  (pad "70" smd rect (at -8 -0.29 180) (size 0.35 2.2) (layers "B.Cu") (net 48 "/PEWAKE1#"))
  (pad "71" smd rect (at -8.25 -0.04 180) (size 0.35 1.7) (layers "F.Cu") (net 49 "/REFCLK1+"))
  (pad "72" smd rect (at -8.5 -0.29 180) (size 0.35 2.2) (layers "B.Cu") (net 10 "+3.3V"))
  (pad "73" smd rect (at -8.75 -0.04 180) (size 0.35 1.7) (layers "F.Cu") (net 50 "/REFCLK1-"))
  (pad "74" smd rect (at -9 -0.29 180) (size 0.35 2.2) (layers "B.Cu") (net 10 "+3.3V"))
  (pad "75" smd rect (at -9.25 -0.04 180) (size 0.35 1.7) (layers "F.Cu") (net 9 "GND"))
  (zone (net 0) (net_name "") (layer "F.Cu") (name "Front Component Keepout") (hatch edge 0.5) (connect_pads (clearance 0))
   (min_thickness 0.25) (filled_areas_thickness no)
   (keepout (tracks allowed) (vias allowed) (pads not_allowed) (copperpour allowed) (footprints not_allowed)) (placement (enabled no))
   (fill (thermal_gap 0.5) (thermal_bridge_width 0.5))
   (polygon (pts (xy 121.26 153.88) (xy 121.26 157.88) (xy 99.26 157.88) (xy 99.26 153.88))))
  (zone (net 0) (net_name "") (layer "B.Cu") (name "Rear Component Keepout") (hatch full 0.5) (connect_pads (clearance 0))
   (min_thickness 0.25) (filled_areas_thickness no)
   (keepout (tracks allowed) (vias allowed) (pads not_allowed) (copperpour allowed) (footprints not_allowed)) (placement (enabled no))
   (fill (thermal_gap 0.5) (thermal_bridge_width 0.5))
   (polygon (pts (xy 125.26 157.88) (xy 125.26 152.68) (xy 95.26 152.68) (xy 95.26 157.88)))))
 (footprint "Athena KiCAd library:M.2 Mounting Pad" (layer "F.Cu") (at 110.26 127.88)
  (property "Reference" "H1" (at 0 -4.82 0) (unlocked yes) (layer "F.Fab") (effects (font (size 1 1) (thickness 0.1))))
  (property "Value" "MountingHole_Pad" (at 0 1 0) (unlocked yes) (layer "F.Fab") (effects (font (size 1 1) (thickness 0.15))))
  (pad "1" thru_hole circle (at 0 0) (size 5.5 5.5) (drill 3.5) (layers "*.Cu" "*.Mask") (remove_unused_layers no) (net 9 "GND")
   (padstack (mode front_inner_back)
    (layer "Inner" (shape circle) (size 5.5 5.5) (zone_connect -1))
    (layer "B.Cu" (shape oval) (size 6 8) (thermal_bridge_angle 45) (zone_connect -1)))))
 (gr_line (start 99.26 127.88) (end 99.26 153.88) (stroke (width 0.1) (type default)) (layer "Edge.Cuts"))
 (gr_line (start 121.26 153.88) (end 121.26 127.88) (stroke (width 0.1) (type default)) (layer "Edge.Cuts"))
 (gr_line (start 121.26 127.88) (end 99.26 127.88) (stroke (width 0.1) (type default)) (layer "Edge.Cuts"))
 (segment (start 103.035 155.429999) (end 103.035 153.900001) (width 0.2) (layer "F.Cu") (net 7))
 (segment (start 103.01 156.73) (end 103.01 155.454999) (width 0.2) (layer "F.Cu") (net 7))
 (segment (start 103.035 153.900001) (end 102.91 153.775001) (width 0.2) (layer "F.Cu") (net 7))
 (segment (start 103.01 155.454999) (end 103.035 155.429999) (width 0.2) (layer "F.Cu") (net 7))
 (segment (start 102.91 153.775001) (end 102.91 153.43) (width 0.2) (layer "F.Cu") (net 7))
 (segment (start 103.485 153.900001) (end 103.61 153.775001) (width 0.2) (layer "F.Cu") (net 5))
 (segment (start 103.485 155.429999) (end 103.485 153.900001) (width 0.2) (layer "F.Cu") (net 5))
 (segment (start 103.51 155.454999) (end 103.485 155.429999) (width 0.2) (layer "F.Cu") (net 5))
 (segment (start 103.61 153.775001) (end 103.61 153.43) (width 0.2) (layer "F.Cu") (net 5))
 (segment (start 103.51 156.73) (end 103.51 155.454999) (width 0.2) (layer "F.Cu") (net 5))
 (segment (start 109.01 156.73) (end 109.01 155.454999) (width 0.2) (layer "F.Cu") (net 1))
 (segment (start 109.01 155.454999) (end 109.035 155.429999) (width 0.2) (layer "F.Cu") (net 1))
 (segment (start 109.035 155.429999) (end 109.035 153.900001) (width 0.2) (layer "F.Cu") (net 1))
 (segment (start 109.035 153.900001) (end 108.91 153.775001) (width 0.2) (layer "F.Cu") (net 1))
 (segment (start 108.91 153.775001) (end 108.91 153.43) (width 0.2) (layer "F.Cu") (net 1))
 (segment (start 109.485 155.429999) (end 109.485 153.900001) (width 0.2) (layer "F.Cu") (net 3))
 (segment (start 109.485 153.900001) (end 109.61 153.775001) (width 0.2) (layer "F.Cu") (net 3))
 (segment (start 109.51 155.454999) (end 109.485 155.429999) (width 0.2) (layer "F.Cu") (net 3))
 (segment (start 109.51 156.73) (end 109.51 155.454999) (width 0.2) (layer "F.Cu") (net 3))
 (segment (start 109.61 153.775001) (end 109.61 153.43) (width 0.2) (layer "F.Cu") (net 3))
 (via (at 115.26 154.11) (size 0.6) (drill 0.3) (layers "F.Cu" "B.Cu") (free yes) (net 9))
 (segment (start 115.26 154.11) (end 115.26 156.48) (width 0.2) (layer "B.Cu") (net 9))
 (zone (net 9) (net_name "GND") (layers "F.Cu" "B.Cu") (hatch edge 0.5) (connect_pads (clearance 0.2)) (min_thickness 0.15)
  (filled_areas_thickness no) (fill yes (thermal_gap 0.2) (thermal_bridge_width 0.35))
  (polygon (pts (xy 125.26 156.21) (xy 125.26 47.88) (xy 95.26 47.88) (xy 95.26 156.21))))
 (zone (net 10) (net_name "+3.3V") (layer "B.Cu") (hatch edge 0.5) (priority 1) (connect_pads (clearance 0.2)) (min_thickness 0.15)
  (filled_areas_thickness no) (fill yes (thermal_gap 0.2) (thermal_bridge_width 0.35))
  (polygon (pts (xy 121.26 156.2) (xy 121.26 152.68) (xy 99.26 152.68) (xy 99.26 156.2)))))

